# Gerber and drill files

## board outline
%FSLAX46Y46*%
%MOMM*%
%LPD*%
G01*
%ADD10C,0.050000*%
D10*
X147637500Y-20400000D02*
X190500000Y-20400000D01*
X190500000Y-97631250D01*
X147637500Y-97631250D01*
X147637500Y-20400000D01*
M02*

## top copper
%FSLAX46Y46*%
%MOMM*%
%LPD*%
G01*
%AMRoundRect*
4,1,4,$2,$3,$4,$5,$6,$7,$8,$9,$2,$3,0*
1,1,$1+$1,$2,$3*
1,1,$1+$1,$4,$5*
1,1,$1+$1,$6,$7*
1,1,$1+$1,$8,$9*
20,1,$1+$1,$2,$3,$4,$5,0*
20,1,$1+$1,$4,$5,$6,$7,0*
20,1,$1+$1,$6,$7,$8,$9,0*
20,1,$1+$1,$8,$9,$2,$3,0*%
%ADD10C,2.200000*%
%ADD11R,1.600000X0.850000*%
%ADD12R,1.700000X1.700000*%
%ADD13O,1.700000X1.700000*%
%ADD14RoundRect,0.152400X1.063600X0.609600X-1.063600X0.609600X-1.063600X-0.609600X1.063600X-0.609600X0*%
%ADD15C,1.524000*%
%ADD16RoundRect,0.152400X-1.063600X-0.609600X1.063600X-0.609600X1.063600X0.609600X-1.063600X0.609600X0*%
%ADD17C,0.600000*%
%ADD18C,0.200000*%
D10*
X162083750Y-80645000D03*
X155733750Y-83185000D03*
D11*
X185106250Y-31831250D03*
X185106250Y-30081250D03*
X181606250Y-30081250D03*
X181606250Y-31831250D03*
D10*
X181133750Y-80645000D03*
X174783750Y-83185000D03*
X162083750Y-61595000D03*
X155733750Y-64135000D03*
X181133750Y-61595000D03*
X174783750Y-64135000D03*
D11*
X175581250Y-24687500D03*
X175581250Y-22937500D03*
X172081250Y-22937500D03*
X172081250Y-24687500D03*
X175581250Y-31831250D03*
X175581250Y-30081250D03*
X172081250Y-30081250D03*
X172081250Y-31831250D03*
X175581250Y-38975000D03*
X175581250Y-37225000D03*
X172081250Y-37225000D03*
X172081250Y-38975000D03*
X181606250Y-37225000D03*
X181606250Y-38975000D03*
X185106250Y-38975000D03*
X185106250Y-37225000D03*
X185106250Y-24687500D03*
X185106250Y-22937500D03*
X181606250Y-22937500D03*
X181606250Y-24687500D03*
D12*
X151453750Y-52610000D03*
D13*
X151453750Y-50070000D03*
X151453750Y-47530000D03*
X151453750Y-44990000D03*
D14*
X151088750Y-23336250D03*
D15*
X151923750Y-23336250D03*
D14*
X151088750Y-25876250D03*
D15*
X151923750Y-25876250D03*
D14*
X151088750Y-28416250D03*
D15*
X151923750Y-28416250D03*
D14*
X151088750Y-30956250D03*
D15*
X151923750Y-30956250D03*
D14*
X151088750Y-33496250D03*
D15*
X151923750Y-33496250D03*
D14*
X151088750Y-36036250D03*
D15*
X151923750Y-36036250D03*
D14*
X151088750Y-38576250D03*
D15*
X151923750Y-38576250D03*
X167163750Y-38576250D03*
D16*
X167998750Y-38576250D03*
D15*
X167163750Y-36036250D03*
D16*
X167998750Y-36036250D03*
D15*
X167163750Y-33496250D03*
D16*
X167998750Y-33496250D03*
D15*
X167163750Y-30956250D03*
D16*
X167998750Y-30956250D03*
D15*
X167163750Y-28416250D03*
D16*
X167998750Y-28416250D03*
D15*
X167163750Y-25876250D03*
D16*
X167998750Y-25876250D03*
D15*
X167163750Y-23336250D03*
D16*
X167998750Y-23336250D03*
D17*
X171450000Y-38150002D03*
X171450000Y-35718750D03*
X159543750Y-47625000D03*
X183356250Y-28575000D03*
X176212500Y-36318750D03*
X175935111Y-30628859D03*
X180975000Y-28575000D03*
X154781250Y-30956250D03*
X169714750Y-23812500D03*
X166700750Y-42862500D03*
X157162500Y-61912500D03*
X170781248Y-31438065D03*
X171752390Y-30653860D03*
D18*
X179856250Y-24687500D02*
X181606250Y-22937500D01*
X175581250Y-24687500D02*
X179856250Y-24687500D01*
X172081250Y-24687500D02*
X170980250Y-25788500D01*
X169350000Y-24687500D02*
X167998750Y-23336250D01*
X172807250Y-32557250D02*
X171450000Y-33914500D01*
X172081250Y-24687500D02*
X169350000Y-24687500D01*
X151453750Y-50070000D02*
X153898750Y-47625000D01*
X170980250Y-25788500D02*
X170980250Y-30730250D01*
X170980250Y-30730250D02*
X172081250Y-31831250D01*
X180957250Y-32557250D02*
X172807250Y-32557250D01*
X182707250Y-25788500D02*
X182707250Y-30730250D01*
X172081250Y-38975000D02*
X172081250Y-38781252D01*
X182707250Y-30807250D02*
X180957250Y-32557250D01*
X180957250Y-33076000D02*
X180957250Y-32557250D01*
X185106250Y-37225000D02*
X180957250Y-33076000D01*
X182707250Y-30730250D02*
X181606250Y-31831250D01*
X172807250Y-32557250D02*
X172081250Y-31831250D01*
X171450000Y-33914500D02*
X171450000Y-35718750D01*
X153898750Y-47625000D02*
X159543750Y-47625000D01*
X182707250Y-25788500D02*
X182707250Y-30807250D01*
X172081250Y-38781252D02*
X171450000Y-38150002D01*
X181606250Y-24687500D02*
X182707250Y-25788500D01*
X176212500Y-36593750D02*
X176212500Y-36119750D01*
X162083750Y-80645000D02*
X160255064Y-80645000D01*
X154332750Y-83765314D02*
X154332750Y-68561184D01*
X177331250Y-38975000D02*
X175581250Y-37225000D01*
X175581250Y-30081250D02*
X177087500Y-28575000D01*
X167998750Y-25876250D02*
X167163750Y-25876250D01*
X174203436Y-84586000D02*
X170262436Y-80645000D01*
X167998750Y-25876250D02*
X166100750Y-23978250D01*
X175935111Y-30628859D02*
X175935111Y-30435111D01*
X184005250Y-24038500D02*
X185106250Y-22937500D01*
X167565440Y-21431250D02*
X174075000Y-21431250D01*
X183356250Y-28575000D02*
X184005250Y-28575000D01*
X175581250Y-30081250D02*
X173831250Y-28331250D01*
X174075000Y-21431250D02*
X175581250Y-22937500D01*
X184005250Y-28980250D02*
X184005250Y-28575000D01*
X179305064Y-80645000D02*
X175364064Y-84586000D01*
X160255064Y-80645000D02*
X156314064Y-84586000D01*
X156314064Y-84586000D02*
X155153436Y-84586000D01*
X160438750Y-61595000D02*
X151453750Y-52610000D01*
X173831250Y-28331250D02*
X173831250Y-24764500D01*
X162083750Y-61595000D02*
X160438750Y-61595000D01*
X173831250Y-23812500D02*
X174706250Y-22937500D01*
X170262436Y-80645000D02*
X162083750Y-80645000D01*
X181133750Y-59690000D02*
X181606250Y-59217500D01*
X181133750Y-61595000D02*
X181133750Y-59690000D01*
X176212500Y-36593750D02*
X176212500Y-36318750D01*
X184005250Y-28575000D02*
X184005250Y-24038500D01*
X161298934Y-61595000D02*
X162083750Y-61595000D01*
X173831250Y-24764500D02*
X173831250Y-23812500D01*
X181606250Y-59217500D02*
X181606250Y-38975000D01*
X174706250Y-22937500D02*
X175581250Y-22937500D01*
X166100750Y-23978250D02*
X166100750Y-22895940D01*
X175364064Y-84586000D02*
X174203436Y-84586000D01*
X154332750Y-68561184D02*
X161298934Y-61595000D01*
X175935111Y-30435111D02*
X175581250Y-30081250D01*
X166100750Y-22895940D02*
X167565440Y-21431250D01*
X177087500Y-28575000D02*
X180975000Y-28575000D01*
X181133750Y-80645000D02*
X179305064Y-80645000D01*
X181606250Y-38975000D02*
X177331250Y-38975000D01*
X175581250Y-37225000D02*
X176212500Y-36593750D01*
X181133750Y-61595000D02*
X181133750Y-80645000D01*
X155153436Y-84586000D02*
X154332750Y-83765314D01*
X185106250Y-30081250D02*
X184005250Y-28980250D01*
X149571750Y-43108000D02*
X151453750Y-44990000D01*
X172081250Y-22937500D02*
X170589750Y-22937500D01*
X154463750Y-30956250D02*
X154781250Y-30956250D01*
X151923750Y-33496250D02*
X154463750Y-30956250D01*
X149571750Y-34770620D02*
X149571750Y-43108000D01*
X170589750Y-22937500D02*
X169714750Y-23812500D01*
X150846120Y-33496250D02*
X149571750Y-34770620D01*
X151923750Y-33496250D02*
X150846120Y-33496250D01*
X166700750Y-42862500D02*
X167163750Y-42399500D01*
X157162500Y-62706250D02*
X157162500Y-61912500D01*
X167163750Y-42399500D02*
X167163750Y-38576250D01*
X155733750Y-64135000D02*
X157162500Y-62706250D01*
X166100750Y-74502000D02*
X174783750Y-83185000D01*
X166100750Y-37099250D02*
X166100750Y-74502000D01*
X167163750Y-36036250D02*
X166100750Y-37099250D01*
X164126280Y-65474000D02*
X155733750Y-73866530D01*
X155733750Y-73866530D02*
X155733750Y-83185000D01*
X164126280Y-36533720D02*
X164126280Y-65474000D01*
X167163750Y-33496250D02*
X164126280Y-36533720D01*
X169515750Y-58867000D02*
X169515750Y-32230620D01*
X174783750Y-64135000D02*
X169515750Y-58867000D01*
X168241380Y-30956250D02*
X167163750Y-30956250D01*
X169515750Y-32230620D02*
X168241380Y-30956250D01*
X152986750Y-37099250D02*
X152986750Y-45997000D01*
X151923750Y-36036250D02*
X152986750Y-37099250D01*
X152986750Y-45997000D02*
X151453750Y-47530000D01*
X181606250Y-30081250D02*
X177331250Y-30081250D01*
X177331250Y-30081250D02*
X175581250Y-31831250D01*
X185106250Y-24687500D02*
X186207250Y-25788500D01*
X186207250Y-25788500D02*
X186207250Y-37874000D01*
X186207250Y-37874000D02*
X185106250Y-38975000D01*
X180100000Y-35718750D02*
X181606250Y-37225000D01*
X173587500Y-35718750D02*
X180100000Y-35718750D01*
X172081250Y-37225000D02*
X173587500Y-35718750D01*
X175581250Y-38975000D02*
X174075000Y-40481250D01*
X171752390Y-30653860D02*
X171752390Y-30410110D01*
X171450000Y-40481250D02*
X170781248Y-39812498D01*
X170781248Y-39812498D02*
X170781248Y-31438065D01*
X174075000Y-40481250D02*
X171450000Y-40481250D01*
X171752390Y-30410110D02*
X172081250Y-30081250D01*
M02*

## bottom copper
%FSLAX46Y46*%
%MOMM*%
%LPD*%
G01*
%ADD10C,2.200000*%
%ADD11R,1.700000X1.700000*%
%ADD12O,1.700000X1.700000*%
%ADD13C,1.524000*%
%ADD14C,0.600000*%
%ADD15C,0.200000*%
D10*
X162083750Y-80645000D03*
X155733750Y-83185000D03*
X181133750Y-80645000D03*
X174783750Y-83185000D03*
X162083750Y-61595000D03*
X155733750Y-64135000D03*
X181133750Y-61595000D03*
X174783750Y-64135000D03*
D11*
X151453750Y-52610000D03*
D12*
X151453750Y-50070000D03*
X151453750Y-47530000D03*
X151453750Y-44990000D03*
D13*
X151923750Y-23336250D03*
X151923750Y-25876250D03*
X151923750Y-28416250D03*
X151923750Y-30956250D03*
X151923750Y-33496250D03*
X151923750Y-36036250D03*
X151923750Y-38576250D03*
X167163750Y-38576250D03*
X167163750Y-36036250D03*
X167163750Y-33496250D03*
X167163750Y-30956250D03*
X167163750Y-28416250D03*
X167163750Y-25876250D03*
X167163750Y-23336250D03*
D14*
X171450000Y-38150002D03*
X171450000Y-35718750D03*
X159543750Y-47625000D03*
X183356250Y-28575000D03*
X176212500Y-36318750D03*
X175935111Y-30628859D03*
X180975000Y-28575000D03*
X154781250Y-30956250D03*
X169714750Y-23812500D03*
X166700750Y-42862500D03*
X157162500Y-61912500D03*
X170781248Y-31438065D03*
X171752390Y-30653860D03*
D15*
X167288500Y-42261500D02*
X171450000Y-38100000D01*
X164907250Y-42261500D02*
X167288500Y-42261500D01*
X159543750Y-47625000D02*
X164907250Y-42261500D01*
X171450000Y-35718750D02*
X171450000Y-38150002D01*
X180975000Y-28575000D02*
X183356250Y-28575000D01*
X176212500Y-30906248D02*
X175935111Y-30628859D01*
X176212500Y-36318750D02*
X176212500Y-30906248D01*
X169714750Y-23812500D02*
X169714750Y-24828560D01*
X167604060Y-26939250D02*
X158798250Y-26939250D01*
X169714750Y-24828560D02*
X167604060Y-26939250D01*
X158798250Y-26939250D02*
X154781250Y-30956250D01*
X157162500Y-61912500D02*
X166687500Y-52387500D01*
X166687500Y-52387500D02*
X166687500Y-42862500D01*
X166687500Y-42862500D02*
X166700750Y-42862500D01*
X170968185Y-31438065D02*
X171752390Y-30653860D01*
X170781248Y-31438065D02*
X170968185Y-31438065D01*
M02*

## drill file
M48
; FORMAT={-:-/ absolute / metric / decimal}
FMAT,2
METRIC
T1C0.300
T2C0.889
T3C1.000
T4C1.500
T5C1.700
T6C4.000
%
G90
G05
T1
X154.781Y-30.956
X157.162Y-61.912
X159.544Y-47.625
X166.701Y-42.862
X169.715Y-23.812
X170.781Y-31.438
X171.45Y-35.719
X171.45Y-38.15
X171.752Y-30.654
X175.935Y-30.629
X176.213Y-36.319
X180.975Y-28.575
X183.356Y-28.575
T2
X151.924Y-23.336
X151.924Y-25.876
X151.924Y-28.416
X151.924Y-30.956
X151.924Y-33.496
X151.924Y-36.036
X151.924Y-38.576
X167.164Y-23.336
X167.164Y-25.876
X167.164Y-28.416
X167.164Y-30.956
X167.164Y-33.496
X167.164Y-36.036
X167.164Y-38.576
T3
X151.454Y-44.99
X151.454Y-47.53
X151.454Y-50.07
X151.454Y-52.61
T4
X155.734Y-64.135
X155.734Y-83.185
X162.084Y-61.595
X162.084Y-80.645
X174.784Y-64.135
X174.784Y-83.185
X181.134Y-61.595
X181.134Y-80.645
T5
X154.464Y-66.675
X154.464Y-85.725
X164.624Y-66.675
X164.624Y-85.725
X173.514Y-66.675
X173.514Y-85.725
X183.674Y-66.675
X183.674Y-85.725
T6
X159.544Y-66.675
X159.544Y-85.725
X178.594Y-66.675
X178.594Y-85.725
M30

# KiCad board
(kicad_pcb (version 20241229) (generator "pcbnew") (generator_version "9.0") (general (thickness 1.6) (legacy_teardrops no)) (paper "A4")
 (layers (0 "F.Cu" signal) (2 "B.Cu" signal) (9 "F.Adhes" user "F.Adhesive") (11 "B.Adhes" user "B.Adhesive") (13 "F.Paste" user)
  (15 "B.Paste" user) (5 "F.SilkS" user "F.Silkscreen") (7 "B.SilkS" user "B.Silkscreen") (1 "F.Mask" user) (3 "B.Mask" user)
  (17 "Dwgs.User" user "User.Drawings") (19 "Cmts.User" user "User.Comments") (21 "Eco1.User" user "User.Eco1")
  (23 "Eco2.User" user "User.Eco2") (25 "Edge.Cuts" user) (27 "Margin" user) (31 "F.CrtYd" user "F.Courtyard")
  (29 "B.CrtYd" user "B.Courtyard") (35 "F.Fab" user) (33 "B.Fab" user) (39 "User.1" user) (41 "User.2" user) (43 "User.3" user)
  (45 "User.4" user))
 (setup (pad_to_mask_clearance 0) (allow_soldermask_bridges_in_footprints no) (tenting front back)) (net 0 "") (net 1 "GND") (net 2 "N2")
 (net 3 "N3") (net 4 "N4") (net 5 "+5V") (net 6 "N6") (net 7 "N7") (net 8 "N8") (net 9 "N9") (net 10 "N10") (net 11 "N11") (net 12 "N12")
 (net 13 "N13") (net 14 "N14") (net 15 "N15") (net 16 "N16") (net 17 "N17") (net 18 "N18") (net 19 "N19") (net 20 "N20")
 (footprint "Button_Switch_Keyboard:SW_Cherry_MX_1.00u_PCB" (layer "F.Cu") (at 162.08375 80.645)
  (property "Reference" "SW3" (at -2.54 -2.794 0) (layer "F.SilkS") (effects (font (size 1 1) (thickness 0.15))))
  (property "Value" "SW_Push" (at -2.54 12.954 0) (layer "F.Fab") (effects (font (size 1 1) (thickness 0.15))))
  (pad "" np_thru_hole circle (at -7.62 5.08) (size 1.7 1.7) (drill 1.7) (layers "*.Cu" "*.Mask"))
  (pad "" np_thru_hole circle (at -2.54 5.08) (size 4 4) (drill 4) (layers "*.Cu" "*.Mask"))
  (pad "" np_thru_hole circle (at 2.54 5.08) (size 1.7 1.7) (drill 1.7) (layers "*.Cu" "*.Mask"))
  (pad "1" thru_hole circle (at 0 0) (size 2.2 2.2) (drill 1.5) (layers "*.Cu" "*.Mask") (remove_unused_layers no) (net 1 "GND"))
  (pad "2" thru_hole circle (at -6.35 2.54) (size 2.2 2.2) (drill 1.5) (layers "*.Cu" "*.Mask") (remove_unused_layers no) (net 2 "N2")))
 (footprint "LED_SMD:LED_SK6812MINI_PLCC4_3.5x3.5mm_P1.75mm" (layer "F.Cu") (at 183.35625 30.95625 180)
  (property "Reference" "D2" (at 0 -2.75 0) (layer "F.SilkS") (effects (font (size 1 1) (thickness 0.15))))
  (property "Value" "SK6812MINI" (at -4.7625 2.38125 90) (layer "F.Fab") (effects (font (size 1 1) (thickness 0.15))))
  (pad "1" smd rect (at -1.75 -0.875 180) (size 1.6 0.85) (layers "F.Cu" "F.Mask" "F.Paste") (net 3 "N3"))
  (pad "2" smd rect (at -1.75 0.875 180) (size 1.6 0.85) (layers "F.Cu" "F.Mask" "F.Paste") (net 1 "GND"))
  (pad "3" smd rect (at 1.75 0.875 180) (size 1.6 0.85) (layers "F.Cu" "F.Mask" "F.Paste") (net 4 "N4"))
  (pad "4" smd rect (at 1.75 -0.875 180) (size 1.6 0.85) (layers "F.Cu" "F.Mask" "F.Paste") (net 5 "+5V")))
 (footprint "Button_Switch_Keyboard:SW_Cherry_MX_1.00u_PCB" (layer "F.Cu") (at 181.13375 80.645)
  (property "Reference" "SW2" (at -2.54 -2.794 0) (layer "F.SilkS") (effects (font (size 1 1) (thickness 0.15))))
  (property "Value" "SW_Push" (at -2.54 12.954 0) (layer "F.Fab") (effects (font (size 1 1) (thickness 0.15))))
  (pad "" np_thru_hole circle (at -7.62 5.08) (size 1.7 1.7) (drill 1.7) (layers "*.Cu" "*.Mask"))
  (pad "" np_thru_hole circle (at -2.54 5.08) (size 4 4) (drill 4) (layers "*.Cu" "*.Mask"))
  (pad "" np_thru_hole circle (at 2.54 5.08) (size 1.7 1.7) (drill 1.7) (layers "*.Cu" "*.Mask"))
  (pad "1" thru_hole circle (at 0 0) (size 2.2 2.2) (drill 1.5) (layers "*.Cu" "*.Mask") (remove_unused_layers no) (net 1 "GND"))
  (pad "2" thru_hole circle (at -6.35 2.54) (size 2.2 2.2) (drill 1.5) (layers "*.Cu" "*.Mask") (remove_unused_layers no) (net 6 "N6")))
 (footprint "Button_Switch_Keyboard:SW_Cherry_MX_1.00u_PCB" (layer "F.Cu") (at 162.08375 61.595)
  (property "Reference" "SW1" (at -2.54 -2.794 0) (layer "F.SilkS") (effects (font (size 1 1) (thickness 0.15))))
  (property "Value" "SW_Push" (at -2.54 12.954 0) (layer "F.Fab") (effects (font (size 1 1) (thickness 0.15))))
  (pad "" np_thru_hole circle (at -7.62 5.08) (size 1.7 1.7) (drill 1.7) (layers "*.Cu" "*.Mask"))
  (pad "" np_thru_hole circle (at -2.54 5.08) (size 4 4) (drill 4) (layers "*.Cu" "*.Mask"))
  (pad "" np_thru_hole circle (at 2.54 5.08) (size 1.7 1.7) (drill 1.7) (layers "*.Cu" "*.Mask"))
  (pad "1" thru_hole circle (at 0 0) (size 2.2 2.2) (drill 1.5) (layers "*.Cu" "*.Mask") (remove_unused_layers no) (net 1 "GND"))
  (pad "2" thru_hole circle (at -6.35 2.54) (size 2.2 2.2) (drill 1.5) (layers "*.Cu" "*.Mask") (remove_unused_layers no) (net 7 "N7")))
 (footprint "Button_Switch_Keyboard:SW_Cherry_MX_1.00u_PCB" (layer "F.Cu") (at 181.13375 61.595)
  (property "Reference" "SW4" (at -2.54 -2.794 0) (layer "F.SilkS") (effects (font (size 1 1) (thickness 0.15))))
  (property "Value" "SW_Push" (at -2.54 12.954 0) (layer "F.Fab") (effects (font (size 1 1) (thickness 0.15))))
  (pad "" np_thru_hole circle (at -7.62 5.08) (size 1.7 1.7) (drill 1.7) (layers "*.Cu" "*.Mask"))
  (pad "" np_thru_hole circle (at -2.54 5.08) (size 4 4) (drill 4) (layers "*.Cu" "*.Mask"))
  (pad "" np_thru_hole circle (at 2.54 5.08) (size 1.7 1.7) (drill 1.7) (layers "*.Cu" "*.Mask"))
  (pad "1" thru_hole circle (at 0 0) (size 2.2 2.2) (drill 1.5) (layers "*.Cu" "*.Mask") (remove_unused_layers no) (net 1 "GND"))
  (pad "2" thru_hole circle (at -6.35 2.54) (size 2.2 2.2) (drill 1.5) (layers "*.Cu" "*.Mask") (remove_unused_layers no) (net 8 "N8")))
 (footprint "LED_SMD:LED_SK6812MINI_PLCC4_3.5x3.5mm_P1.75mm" (layer "F.Cu") (at 173.83125 23.8125 180)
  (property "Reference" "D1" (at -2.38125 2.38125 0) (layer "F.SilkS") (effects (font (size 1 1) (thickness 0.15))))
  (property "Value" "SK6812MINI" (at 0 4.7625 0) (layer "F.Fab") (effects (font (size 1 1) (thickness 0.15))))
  (pad "1" smd rect (at -1.75 -0.875 180) (size 1.6 0.85) (layers "F.Cu" "F.Mask" "F.Paste") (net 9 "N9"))
  (pad "2" smd rect (at -1.75 0.875 180) (size 1.6 0.85) (layers "F.Cu" "F.Mask" "F.Paste") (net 1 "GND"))
  (pad "3" smd rect (at 1.75 0.875 180) (size 1.6 0.85) (layers "F.Cu" "F.Mask" "F.Paste") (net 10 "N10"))
  (pad "4" smd rect (at 1.75 -0.875 180) (size 1.6 0.85) (layers "F.Cu" "F.Mask" "F.Paste") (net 5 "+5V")))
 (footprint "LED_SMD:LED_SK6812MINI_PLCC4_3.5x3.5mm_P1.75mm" (layer "F.Cu") (at 173.83125 30.95625 180)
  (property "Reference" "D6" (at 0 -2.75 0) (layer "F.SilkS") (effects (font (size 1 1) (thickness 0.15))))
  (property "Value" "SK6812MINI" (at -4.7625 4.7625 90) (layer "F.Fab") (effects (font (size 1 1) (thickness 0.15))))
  (pad "1" smd rect (at -1.75 -0.875 180) (size 1.6 0.85) (layers "F.Cu" "F.Mask" "F.Paste") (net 4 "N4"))
  (pad "2" smd rect (at -1.75 0.875 180) (size 1.6 0.85) (layers "F.Cu" "F.Mask" "F.Paste") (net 1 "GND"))
  (pad "3" smd rect (at 1.75 0.875 180) (size 1.6 0.85) (layers "F.Cu" "F.Mask" "F.Paste") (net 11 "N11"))
  (pad "4" smd rect (at 1.75 -0.875 180) (size 1.6 0.85) (layers "F.Cu" "F.Mask" "F.Paste") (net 5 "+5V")))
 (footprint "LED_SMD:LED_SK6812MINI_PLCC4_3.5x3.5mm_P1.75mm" (layer "F.Cu") (at 173.83125 38.1 180)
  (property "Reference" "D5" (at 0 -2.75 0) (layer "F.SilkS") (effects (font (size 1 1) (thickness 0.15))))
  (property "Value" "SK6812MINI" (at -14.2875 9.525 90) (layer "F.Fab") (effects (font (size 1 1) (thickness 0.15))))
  (pad "1" smd rect (at -1.75 -0.875 180) (size 1.6 0.85) (layers "F.Cu" "F.Mask" "F.Paste") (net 11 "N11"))
  (pad "2" smd rect (at -1.75 0.875 180) (size 1.6 0.85) (layers "F.Cu" "F.Mask" "F.Paste") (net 1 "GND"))
  (pad "3" smd rect (at 1.75 0.875 180) (size 1.6 0.85) (layers "F.Cu" "F.Mask" "F.Paste") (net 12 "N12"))
  (pad "4" smd rect (at 1.75 -0.875 180) (size 1.6 0.85) (layers "F.Cu" "F.Mask" "F.Paste") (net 5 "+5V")))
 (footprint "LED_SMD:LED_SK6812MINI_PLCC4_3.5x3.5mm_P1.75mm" (layer "F.Cu") (at 183.35625 38.1)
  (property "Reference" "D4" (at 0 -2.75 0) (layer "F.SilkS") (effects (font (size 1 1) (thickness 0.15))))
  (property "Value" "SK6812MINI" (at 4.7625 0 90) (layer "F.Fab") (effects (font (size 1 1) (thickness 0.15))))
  (pad "1" smd rect (at -1.75 -0.875) (size 1.6 0.85) (layers "F.Cu" "F.Mask" "F.Paste") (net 12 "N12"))
  (pad "2" smd rect (at -1.75 0.875) (size 1.6 0.85) (layers "F.Cu" "F.Mask" "F.Paste") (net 1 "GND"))
  (pad "3" smd rect (at 1.75 0.875) (size 1.6 0.85) (layers "F.Cu" "F.Mask" "F.Paste") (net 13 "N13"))
  (pad "4" smd rect (at 1.75 -0.875) (size 1.6 0.85) (layers "F.Cu" "F.Mask" "F.Paste") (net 5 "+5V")))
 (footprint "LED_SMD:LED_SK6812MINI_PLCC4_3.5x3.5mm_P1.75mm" (layer "F.Cu") (at 183.35625 23.8125 180)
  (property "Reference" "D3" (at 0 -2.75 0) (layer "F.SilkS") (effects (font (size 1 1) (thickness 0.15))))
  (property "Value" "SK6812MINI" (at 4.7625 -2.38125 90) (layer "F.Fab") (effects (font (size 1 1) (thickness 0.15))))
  (pad "1" smd rect (at -1.75 -0.875 180) (size 1.6 0.85) (layers "F.Cu" "F.Mask" "F.Paste") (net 13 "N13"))
  (pad "2" smd rect (at -1.75 0.875 180) (size 1.6 0.85) (layers "F.Cu" "F.Mask" "F.Paste") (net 1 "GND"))
  (pad "3" smd rect (at 1.75 0.875 180) (size 1.6 0.85) (layers "F.Cu" "F.Mask" "F.Paste") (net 9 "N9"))
  (pad "4" smd rect (at 1.75 -0.875 180) (size 1.6 0.85) (layers "F.Cu" "F.Mask" "F.Paste") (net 5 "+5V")))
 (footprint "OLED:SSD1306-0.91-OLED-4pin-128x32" (layer "F.Cu") (at 187.95375 54.8 180)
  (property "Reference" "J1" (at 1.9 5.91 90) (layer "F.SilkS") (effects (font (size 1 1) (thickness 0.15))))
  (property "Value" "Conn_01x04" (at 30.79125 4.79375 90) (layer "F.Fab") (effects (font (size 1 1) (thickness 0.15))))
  (pad "1" thru_hole rect (at 36.5 2.19 180) (size 1.7 1.7) (drill 1) (layers "*.Cu" "*.Mask") (remove_unused_layers no) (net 1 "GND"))
  (pad "2" thru_hole oval (at 36.5 4.73 180) (size 1.7 1.7) (drill 1) (layers "*.Cu" "*.Mask") (remove_unused_layers no) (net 5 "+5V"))
  (pad "3" thru_hole oval (at 36.5 7.27 180) (size 1.7 1.7) (drill 1) (layers "*.Cu" "*.Mask") (remove_unused_layers no) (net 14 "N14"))
  (pad "4" thru_hole oval (at 36.5 9.81 180) (size 1.7 1.7) (drill 1) (layers "*.Cu" "*.Mask") (remove_unused_layers no) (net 10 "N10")))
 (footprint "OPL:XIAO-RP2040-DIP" (layer "F.Cu") (at 159.54375 30.95625)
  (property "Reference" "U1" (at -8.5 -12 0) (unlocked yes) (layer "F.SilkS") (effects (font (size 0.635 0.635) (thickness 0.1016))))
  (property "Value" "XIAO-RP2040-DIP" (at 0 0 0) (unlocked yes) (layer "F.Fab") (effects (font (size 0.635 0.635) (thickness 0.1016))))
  (pad "1" smd roundrect (at -8.455 -7.62 180) (size 2.432 1.524) (layers "F.Cu" "F.Mask") (roundrect_rratio 0.1) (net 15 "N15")
   (thermal_bridge_angle 45))
  (pad "1" thru_hole circle (at -7.62 -7.62 180) (size 1.524 1.524) (drill 0.889) (layers "*.Cu" "*.Mask") (remove_unused_layers no)
   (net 15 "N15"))
  (pad "2" smd roundrect (at -8.455 -5.08 180) (size 2.432 1.524) (layers "F.Cu" "F.Mask") (roundrect_rratio 0.1) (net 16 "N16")
   (thermal_bridge_angle 45))
  (pad "2" thru_hole circle (at -7.62 -5.08 180) (size 1.524 1.524) (drill 0.889) (layers "*.Cu" "*.Mask") (remove_unused_layers no)
   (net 16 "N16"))
  (pad "3" smd roundrect (at -8.455 -2.54 180) (size 2.432 1.524) (layers "F.Cu" "F.Mask") (roundrect_rratio 0.1) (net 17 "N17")
   (thermal_bridge_angle 45))
  (pad "3" thru_hole circle (at -7.62 -2.54 180) (size 1.524 1.524) (drill 0.889) (layers "*.Cu" "*.Mask") (remove_unused_layers no)
   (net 17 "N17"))
  (pad "4" smd roundrect (at -8.455 0 180) (size 2.432 1.524) (layers "F.Cu" "F.Mask") (roundrect_rratio 0.1) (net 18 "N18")
   (thermal_bridge_angle 45))
  (pad "4" thru_hole circle (at -7.62 0 180) (size 1.524 1.524) (drill 0.889) (layers "*.Cu" "*.Mask") (remove_unused_layers no)
   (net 18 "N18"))
  (pad "5" smd roundrect (at -8.455 2.54 180) (size 2.432 1.524) (layers "F.Cu" "F.Mask") (roundrect_rratio 0.1) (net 10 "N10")
   (thermal_bridge_angle 45))
  (pad "5" thru_hole circle (at -7.62 2.54 180) (size 1.524 1.524) (drill 0.889) (layers "*.Cu" "*.Mask") (remove_unused_layers no)
   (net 10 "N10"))
  (pad "6" smd roundrect (at -8.455 5.08 180) (size 2.432 1.524) (layers "F.Cu" "F.Mask") (roundrect_rratio 0.1) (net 14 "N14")
   (thermal_bridge_angle 45))
  (pad "6" thru_hole circle (at -7.62 5.08 180) (size 1.524 1.524) (drill 0.889) (layers "*.Cu" "*.Mask") (remove_unused_layers no)
   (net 14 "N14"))
  (pad "7" smd roundrect (at -8.455 7.62 180) (size 2.432 1.524) (layers "F.Cu" "F.Mask") (roundrect_rratio 0.1) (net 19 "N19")
   (thermal_bridge_angle 45))
  (pad "7" thru_hole circle (at -7.62 7.62 180) (size 1.524 1.524) (drill 0.889) (layers "*.Cu" "*.Mask") (remove_unused_layers no)
   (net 19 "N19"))
  (pad "8" thru_hole circle (at 7.62 7.62) (size 1.524 1.524) (drill 0.889) (layers "*.Cu" "*.Mask") (remove_unused_layers no) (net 7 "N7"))
  (pad "8" smd roundrect (at 8.455 7.62) (size 2.432 1.524) (layers "F.Cu" "F.Mask") (roundrect_rratio 0.1) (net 7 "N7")
   (thermal_bridge_angle 45))
  (pad "9" thru_hole circle (at 7.62 5.08) (size 1.524 1.524) (drill 0.889) (layers "*.Cu" "*.Mask") (remove_unused_layers no) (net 6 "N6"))
  (pad "9" smd roundrect (at 8.455 5.08) (size 2.432 1.524) (layers "F.Cu" "F.Mask") (roundrect_rratio 0.1) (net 6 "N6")
   (thermal_bridge_angle 45))
  (pad "10" thru_hole circle (at 7.62 2.54) (size 1.524 1.524) (drill 0.889) (layers "*.Cu" "*.Mask") (remove_unused_layers no) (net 2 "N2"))
  (pad "10" smd roundrect (at 8.455 2.54) (size 2.432 1.524) (layers "F.Cu" "F.Mask") (roundrect_rratio 0.1) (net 2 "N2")
   (thermal_bridge_angle 45))
  (pad "11" thru_hole circle (at 7.62 0) (size 1.524 1.524) (drill 0.889) (layers "*.Cu" "*.Mask") (remove_unused_layers no) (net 8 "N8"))
  (pad "11" smd roundrect (at 8.455 0) (size 2.432 1.524) (layers "F.Cu" "F.Mask") (roundrect_rratio 0.1) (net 8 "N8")
   (thermal_bridge_angle 45))
  (pad "12" thru_hole circle (at 7.62 -2.54) (size 1.524 1.524) (drill 0.889) (layers "*.Cu" "*.Mask") (remove_unused_layers no)
   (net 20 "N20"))
  (pad "12" smd roundrect (at 8.455 -2.54) (size 2.432 1.524) (layers "F.Cu" "F.Mask") (roundrect_rratio 0.1) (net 20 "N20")
   (thermal_bridge_angle 45))
  (pad "13" thru_hole circle (at 7.62 -5.08) (size 1.524 1.524) (drill 0.889) (layers "*.Cu" "*.Mask") (remove_unused_layers no)
   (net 1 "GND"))
  (pad "13" smd roundrect (at 8.455 -5.08) (size 2.432 1.524) (layers "F.Cu" "F.Mask") (roundrect_rratio 0.1) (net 1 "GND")
   (thermal_bridge_angle 45))
  (pad "14" thru_hole circle (at 7.62 -7.62) (size 1.524 1.524) (drill 0.889) (layers "*.Cu" "*.Mask") (remove_unused_layers no)
   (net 5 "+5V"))
  (pad "14" smd roundrect (at 8.455 -7.62) (size 2.432 1.524) (layers "F.Cu" "F.Mask") (roundrect_rratio 0.1) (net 5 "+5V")
   (thermal_bridge_angle 45)))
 (gr_rect (start 147.6375 20.4) (end 190.5 97.63125) (stroke (width 0.05) (type solid)) (fill no) (layer "Edge.Cuts"))
 (segment (start 179.85625 24.6875) (end 181.60625 22.9375) (width 0.2) (layer "F.Cu") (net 9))
 (segment (start 175.58125 24.6875) (end 179.85625 24.6875) (width 0.2) (layer "F.Cu") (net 9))
 (segment (start 172.08125 24.6875) (end 170.98025 25.7885) (width 0.2) (layer "F.Cu") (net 5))
 (segment (start 169.35 24.6875) (end 167.99875 23.33625) (width 0.2) (layer "F.Cu") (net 5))
 (segment (start 172.80725 32.55725) (end 171.45 33.9145) (width 0.2) (layer "F.Cu") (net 5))
 (segment (start 172.08125 24.6875) (end 169.35 24.6875) (width 0.2) (layer "F.Cu") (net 5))
 (segment (start 151.45375 50.07) (end 153.89875 47.625) (width 0.2) (layer "F.Cu") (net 5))
 (segment (start 170.98025 25.7885) (end 170.98025 30.73025) (width 0.2) (layer "F.Cu") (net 5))
 (segment (start 170.98025 30.73025) (end 172.08125 31.83125) (width 0.2) (layer "F.Cu") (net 5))
 (segment (start 180.95725 32.55725) (end 172.80725 32.55725) (width 0.2) (layer "F.Cu") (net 5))
 (segment (start 182.70725 25.7885) (end 182.70725 30.73025) (width 0.2) (layer "F.Cu") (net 5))
 (segment (start 172.08125 38.975) (end 172.08125 38.781252) (width 0.2) (layer "F.Cu") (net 5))
 (segment (start 182.70725 30.80725) (end 180.95725 32.55725) (width 0.2) (layer "F.Cu") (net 5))
 (segment (start 180.95725 33.076) (end 180.95725 32.55725) (width 0.2) (layer "F.Cu") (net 5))
 (segment (start 185.10625 37.225) (end 180.95725 33.076) (width 0.2) (layer "F.Cu") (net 5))
 (segment (start 182.70725 30.73025) (end 181.60625 31.83125) (width 0.2) (layer "F.Cu") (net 5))
 (segment (start 172.80725 32.55725) (end 172.08125 31.83125) (width 0.2) (layer "F.Cu") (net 5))
 (segment (start 171.45 33.9145) (end 171.45 35.71875) (width 0.2) (layer "F.Cu") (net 5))
 (segment (start 153.89875 47.625) (end 159.54375 47.625) (width 0.2) (layer "F.Cu") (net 5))
 (segment (start 182.70725 25.7885) (end 182.70725 30.80725) (width 0.2) (layer "F.Cu") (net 5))
 (segment (start 172.08125 38.781252) (end 171.45 38.150002) (width 0.2) (layer "F.Cu") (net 5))
 (segment (start 181.60625 24.6875) (end 182.70725 25.7885) (width 0.2) (layer "F.Cu") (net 5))
 (via (at 171.45 38.150002) (size 0.6) (drill 0.3) (layers "F.Cu" "B.Cu") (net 5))
 (via (at 171.45 35.71875) (size 0.6) (drill 0.3) (layers "F.Cu" "B.Cu") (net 5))
 (via (at 159.54375 47.625) (size 0.6) (drill 0.3) (layers "F.Cu" "B.Cu") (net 5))
 (segment (start 167.2885 42.2615) (end 171.45 38.1) (width 0.2) (layer "B.Cu") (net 5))
 (segment (start 164.90725 42.2615) (end 167.2885 42.2615) (width 0.2) (layer "B.Cu") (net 5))
 (segment (start 159.54375 47.625) (end 164.90725 42.2615) (width 0.2) (layer "B.Cu") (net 5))
 (segment (start 171.45 35.71875) (end 171.45 38.150002) (width 0.2) (layer "B.Cu") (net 5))
 (segment (start 176.2125 36.59375) (end 176.2125 36.11975) (width 0.2) (layer "F.Cu") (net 1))
 (segment (start 162.08375 80.645) (end 160.255064 80.645) (width 0.2) (layer "F.Cu") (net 1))
 (segment (start 154.33275 83.765314) (end 154.33275 68.561184) (width 0.2) (layer "F.Cu") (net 1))
 (segment (start 177.33125 38.975) (end 175.58125 37.225) (width 0.2) (layer "F.Cu") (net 1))
 (segment (start 175.58125 30.08125) (end 177.0875 28.575) (width 0.2) (layer "F.Cu") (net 1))
 (segment (start 167.99875 25.87625) (end 167.16375 25.87625) (width 0.2) (layer "F.Cu") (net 1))
 (segment (start 174.203436 84.586) (end 170.262436 80.645) (width 0.2) (layer "F.Cu") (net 1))
 (segment (start 167.99875 25.87625) (end 166.10075 23.97825) (width 0.2) (layer "F.Cu") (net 1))
 (segment (start 175.935111 30.628859) (end 175.935111 30.435111) (width 0.2) (layer "F.Cu") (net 1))
 (segment (start 184.00525 24.0385) (end 185.10625 22.9375) (width 0.2) (layer "F.Cu") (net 1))
 (segment (start 167.56544 21.43125) (end 174.075 21.43125) (width 0.2) (layer "F.Cu") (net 1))
 (segment (start 183.35625 28.575) (end 184.00525 28.575) (width 0.2) (layer "F.Cu") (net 1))
 (segment (start 175.58125 30.08125) (end 173.83125 28.33125) (width 0.2) (layer "F.Cu") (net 1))
 (segment (start 174.075 21.43125) (end 175.58125 22.9375) (width 0.2) (layer "F.Cu") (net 1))
 (segment (start 184.00525 28.98025) (end 184.00525 28.575) (width 0.2) (layer "F.Cu") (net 1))
 (segment (start 179.305064 80.645) (end 175.364064 84.586) (width 0.2) (layer "F.Cu") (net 1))
 (segment (start 160.255064 80.645) (end 156.314064 84.586) (width 0.2) (layer "F.Cu") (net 1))
 (segment (start 156.314064 84.586) (end 155.153436 84.586) (width 0.2) (layer "F.Cu") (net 1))
 (segment (start 160.43875 61.595) (end 151.45375 52.61) (width 0.2) (layer "F.Cu") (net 1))
 (segment (start 173.83125 28.33125) (end 173.83125 24.7645) (width 0.2) (layer "F.Cu") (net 1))
 (segment (start 162.08375 61.595) (end 160.43875 61.595) (width 0.2) (layer "F.Cu") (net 1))
 (segment (start 173.83125 23.8125) (end 174.70625 22.9375) (width 0.2) (layer "F.Cu") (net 1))
 (segment (start 170.262436 80.645) (end 162.08375 80.645) (width 0.2) (layer "F.Cu") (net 1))
 (segment (start 181.13375 59.69) (end 181.60625 59.2175) (width 0.2) (layer "F.Cu") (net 1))
 (segment (start 181.13375 61.595) (end 181.13375 59.69) (width 0.2) (layer "F.Cu") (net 1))
 (segment (start 176.2125 36.59375) (end 176.2125 36.31875) (width 0.2) (layer "F.Cu") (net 1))
 (segment (start 184.00525 28.575) (end 184.00525 24.0385) (width 0.2) (layer "F.Cu") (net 1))
 (segment (start 161.298934 61.595) (end 162.08375 61.595) (width 0.2) (layer "F.Cu") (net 1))
 (segment (start 173.83125 24.7645) (end 173.83125 23.8125) (width 0.2) (layer "F.Cu") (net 1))
 (segment (start 181.60625 59.2175) (end 181.60625 38.975) (width 0.2) (layer "F.Cu") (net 1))
 (segment (start 174.70625 22.9375) (end 175.58125 22.9375) (width 0.2) (layer "F.Cu") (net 1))
 (segment (start 166.10075 23.97825) (end 166.10075 22.89594) (width 0.2) (layer "F.Cu") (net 1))
 (segment (start 175.364064 84.586) (end 174.203436 84.586) (width 0.2) (layer "F.Cu") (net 1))
 (segment (start 154.33275 68.561184) (end 161.298934 61.595) (width 0.2) (layer "F.Cu") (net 1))
 (segment (start 175.935111 30.435111) (end 175.58125 30.08125) (width 0.2) (layer "F.Cu") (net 1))
 (segment (start 166.10075 22.89594) (end 167.56544 21.43125) (width 0.2) (layer "F.Cu") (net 1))
 (segment (start 177.0875 28.575) (end 180.975 28.575) (width 0.2) (layer "F.Cu") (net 1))
 (segment (start 181.13375 80.645) (end 179.305064 80.645) (width 0.2) (layer "F.Cu") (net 1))
 (segment (start 181.60625 38.975) (end 177.33125 38.975) (width 0.2) (layer "F.Cu") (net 1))
 (segment (start 175.58125 37.225) (end 176.2125 36.59375) (width 0.2) (layer "F.Cu") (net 1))
 (segment (start 181.13375 61.595) (end 181.13375 80.645) (width 0.2) (layer "F.Cu") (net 1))
 (segment (start 155.153436 84.586) (end 154.33275 83.765314) (width 0.2) (layer "F.Cu") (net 1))
 (segment (start 185.10625 30.08125) (end 184.00525 28.98025) (width 0.2) (layer "F.Cu") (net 1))
 (via (at 183.35625 28.575) (size 0.6) (drill 0.3) (layers "F.Cu" "B.Cu") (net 1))
 (via (at 176.2125 36.31875) (size 0.6) (drill 0.3) (layers "F.Cu" "B.Cu") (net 1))
 (via (at 175.935111 30.628859) (size 0.6) (drill 0.3) (layers "F.Cu" "B.Cu") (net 1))
 (via (at 180.975 28.575) (size 0.6) (drill 0.3) (layers "F.Cu" "B.Cu") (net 1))
 (segment (start 180.975 28.575) (end 183.35625 28.575) (width 0.2) (layer "B.Cu") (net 1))
 (segment (start 176.2125 30.906248) (end 175.935111 30.628859) (width 0.2) (layer "B.Cu") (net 1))
 (segment (start 176.2125 36.31875) (end 176.2125 30.906248) (width 0.2) (layer "B.Cu") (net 1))
 (segment (start 149.57175 43.108) (end 151.45375 44.99) (width 0.2) (layer "F.Cu") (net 10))
 (segment (start 172.08125 22.9375) (end 170.58975 22.9375) (width 0.2) (layer "F.Cu") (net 10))
 (segment (start 154.46375 30.95625) (end 154.78125 30.95625) (width 0.2) (layer "F.Cu") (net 10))
 (segment (start 151.92375 33.49625) (end 154.46375 30.95625) (width 0.2) (layer "F.Cu") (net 10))
 (segment (start 149.57175 34.77062) (end 149.57175 43.108) (width 0.2) (layer "F.Cu") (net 10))
 (segment (start 170.58975 22.9375) (end 169.71475 23.8125) (width 0.2) (layer "F.Cu") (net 10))
 (segment (start 150.84612 33.49625) (end 149.57175 34.77062) (width 0.2) (layer "F.Cu") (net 10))
 (segment (start 151.92375 33.49625) (end 150.84612 33.49625) (width 0.2) (layer "F.Cu") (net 10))
 (via (at 154.78125 30.95625) (size 0.6) (drill 0.3) (layers "F.Cu" "B.Cu") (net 10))
 (via (at 169.71475 23.8125) (size 0.6) (drill 0.3) (layers "F.Cu" "B.Cu") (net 10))
 (segment (start 169.71475 23.8125) (end 169.71475 24.82856) (width 0.2) (layer "B.Cu") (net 10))
 (segment (start 167.60406 26.93925) (end 158.79825 26.93925) (width 0.2) (layer "B.Cu") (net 10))
 (segment (start 169.71475 24.82856) (end 167.60406 26.93925) (width 0.2) (layer "B.Cu") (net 10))
 (segment (start 158.79825 26.93925) (end 154.78125 30.95625) (width 0.2) (layer "B.Cu") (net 10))
 (segment (start 166.70075 42.8625) (end 167.16375 42.3995) (width 0.2) (layer "F.Cu") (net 7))
 (segment (start 157.1625 62.70625) (end 157.1625 61.9125) (width 0.2) (layer "F.Cu") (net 7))
 (segment (start 167.16375 42.3995) (end 167.16375 38.57625) (width 0.2) (layer "F.Cu") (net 7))
 (segment (start 155.73375 64.135) (end 157.1625 62.70625) (width 0.2) (layer "F.Cu") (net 7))
 (via (at 166.70075 42.8625) (size 0.6) (drill 0.3) (layers "F.Cu" "B.Cu") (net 7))
 (via (at 157.1625 61.9125) (size 0.6) (drill 0.3) (layers "F.Cu" "B.Cu") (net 7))
 (segment (start 157.1625 61.9125) (end 166.6875 52.3875) (width 0.2) (layer "B.Cu") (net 7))
 (segment (start 166.6875 52.3875) (end 166.6875 42.8625) (width 0.2) (layer "B.Cu") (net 7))
 (segment (start 166.6875 42.8625) (end 166.70075 42.8625) (width 0.2) (layer "B.Cu") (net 7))
 (segment (start 166.10075 74.502) (end 174.78375 83.185) (width 0.2) (layer "F.Cu") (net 6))
 (segment (start 166.10075 37.09925) (end 166.10075 74.502) (width 0.2) (layer "F.Cu") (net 6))
 (segment (start 167.16375 36.03625) (end 166.10075 37.09925) (width 0.2) (layer "F.Cu") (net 6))
 (segment (start 164.12628 65.474) (end 155.73375 73.86653) (width 0.2) (layer "F.Cu") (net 2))
 (segment (start 155.73375 73.86653) (end 155.73375 83.185) (width 0.2) (layer "F.Cu") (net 2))
 (segment (start 164.12628 36.53372) (end 164.12628 65.474) (width 0.2) (layer "F.Cu") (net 2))
 (segment (start 167.16375 33.49625) (end 164.12628 36.53372) (width 0.2) (layer "F.Cu") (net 2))
 (segment (start 169.51575 58.867) (end 169.51575 32.23062) (width 0.2) (layer "F.Cu") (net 8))
 (segment (start 174.78375 64.135) (end 169.51575 58.867) (width 0.2) (layer "F.Cu") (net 8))
 (segment (start 168.24138 30.95625) (end 167.16375 30.95625) (width 0.2) (layer "F.Cu") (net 8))
 (segment (start 169.51575 32.23062) (end 168.24138 30.95625) (width 0.2) (layer "F.Cu") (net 8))
 (segment (start 152.98675 37.09925) (end 152.98675 45.997) (width 0.2) (layer "F.Cu") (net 14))
 (segment (start 151.92375 36.03625) (end 152.98675 37.09925) (width 0.2) (layer "F.Cu") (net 14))
 (segment (start 152.98675 45.997) (end 151.45375 47.53) (width 0.2) (layer "F.Cu") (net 14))
 (segment (start 181.60625 30.08125) (end 177.33125 30.08125) (width 0.2) (layer "F.Cu") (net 4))
 (segment (start 177.33125 30.08125) (end 175.58125 31.83125) (width 0.2) (layer "F.Cu") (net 4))
 (segment (start 185.10625 24.6875) (end 186.20725 25.7885) (width 0.2) (layer "F.Cu") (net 13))
 (segment (start 186.20725 25.7885) (end 186.20725 37.874) (width 0.2) (layer "F.Cu") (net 13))
 (segment (start 186.20725 37.874) (end 185.10625 38.975) (width 0.2) (layer "F.Cu") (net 13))
 (segment (start 180.1 35.71875) (end 181.60625 37.225) (width 0.2) (layer "F.Cu") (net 12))
 (segment (start 173.5875 35.71875) (end 180.1 35.71875) (width 0.2) (layer "F.Cu") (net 12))
 (segment (start 172.08125 37.225) (end 173.5875 35.71875) (width 0.2) (layer "F.Cu") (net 12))
 (segment (start 175.58125 38.975) (end 174.075 40.48125) (width 0.2) (layer "F.Cu") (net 11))
 (segment (start 171.75239 30.65386) (end 171.75239 30.41011) (width 0.2) (layer "F.Cu") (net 11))
 (segment (start 171.45 40.48125) (end 170.781248 39.812498) (width 0.2) (layer "F.Cu") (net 11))
 (segment (start 170.781248 39.812498) (end 170.781248 31.438065) (width 0.2) (layer "F.Cu") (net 11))
 (segment (start 174.075 40.48125) (end 171.45 40.48125) (width 0.2) (layer "F.Cu") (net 11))
 (segment (start 171.75239 30.41011) (end 172.08125 30.08125) (width 0.2) (layer "F.Cu") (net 11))
 (via (at 170.781248 31.438065) (size 0.6) (drill 0.3) (layers "F.Cu" "B.Cu") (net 11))
 (via (at 171.75239 30.65386) (size 0.6) (drill 0.3) (layers "F.Cu" "B.Cu") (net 11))
 (segment (start 170.968185 31.438065) (end 171.75239 30.65386) (width 0.2) (layer "B.Cu") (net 11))
 (segment (start 170.781248 31.438065) (end 170.968185 31.438065) (width 0.2) (layer "B.Cu") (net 11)))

